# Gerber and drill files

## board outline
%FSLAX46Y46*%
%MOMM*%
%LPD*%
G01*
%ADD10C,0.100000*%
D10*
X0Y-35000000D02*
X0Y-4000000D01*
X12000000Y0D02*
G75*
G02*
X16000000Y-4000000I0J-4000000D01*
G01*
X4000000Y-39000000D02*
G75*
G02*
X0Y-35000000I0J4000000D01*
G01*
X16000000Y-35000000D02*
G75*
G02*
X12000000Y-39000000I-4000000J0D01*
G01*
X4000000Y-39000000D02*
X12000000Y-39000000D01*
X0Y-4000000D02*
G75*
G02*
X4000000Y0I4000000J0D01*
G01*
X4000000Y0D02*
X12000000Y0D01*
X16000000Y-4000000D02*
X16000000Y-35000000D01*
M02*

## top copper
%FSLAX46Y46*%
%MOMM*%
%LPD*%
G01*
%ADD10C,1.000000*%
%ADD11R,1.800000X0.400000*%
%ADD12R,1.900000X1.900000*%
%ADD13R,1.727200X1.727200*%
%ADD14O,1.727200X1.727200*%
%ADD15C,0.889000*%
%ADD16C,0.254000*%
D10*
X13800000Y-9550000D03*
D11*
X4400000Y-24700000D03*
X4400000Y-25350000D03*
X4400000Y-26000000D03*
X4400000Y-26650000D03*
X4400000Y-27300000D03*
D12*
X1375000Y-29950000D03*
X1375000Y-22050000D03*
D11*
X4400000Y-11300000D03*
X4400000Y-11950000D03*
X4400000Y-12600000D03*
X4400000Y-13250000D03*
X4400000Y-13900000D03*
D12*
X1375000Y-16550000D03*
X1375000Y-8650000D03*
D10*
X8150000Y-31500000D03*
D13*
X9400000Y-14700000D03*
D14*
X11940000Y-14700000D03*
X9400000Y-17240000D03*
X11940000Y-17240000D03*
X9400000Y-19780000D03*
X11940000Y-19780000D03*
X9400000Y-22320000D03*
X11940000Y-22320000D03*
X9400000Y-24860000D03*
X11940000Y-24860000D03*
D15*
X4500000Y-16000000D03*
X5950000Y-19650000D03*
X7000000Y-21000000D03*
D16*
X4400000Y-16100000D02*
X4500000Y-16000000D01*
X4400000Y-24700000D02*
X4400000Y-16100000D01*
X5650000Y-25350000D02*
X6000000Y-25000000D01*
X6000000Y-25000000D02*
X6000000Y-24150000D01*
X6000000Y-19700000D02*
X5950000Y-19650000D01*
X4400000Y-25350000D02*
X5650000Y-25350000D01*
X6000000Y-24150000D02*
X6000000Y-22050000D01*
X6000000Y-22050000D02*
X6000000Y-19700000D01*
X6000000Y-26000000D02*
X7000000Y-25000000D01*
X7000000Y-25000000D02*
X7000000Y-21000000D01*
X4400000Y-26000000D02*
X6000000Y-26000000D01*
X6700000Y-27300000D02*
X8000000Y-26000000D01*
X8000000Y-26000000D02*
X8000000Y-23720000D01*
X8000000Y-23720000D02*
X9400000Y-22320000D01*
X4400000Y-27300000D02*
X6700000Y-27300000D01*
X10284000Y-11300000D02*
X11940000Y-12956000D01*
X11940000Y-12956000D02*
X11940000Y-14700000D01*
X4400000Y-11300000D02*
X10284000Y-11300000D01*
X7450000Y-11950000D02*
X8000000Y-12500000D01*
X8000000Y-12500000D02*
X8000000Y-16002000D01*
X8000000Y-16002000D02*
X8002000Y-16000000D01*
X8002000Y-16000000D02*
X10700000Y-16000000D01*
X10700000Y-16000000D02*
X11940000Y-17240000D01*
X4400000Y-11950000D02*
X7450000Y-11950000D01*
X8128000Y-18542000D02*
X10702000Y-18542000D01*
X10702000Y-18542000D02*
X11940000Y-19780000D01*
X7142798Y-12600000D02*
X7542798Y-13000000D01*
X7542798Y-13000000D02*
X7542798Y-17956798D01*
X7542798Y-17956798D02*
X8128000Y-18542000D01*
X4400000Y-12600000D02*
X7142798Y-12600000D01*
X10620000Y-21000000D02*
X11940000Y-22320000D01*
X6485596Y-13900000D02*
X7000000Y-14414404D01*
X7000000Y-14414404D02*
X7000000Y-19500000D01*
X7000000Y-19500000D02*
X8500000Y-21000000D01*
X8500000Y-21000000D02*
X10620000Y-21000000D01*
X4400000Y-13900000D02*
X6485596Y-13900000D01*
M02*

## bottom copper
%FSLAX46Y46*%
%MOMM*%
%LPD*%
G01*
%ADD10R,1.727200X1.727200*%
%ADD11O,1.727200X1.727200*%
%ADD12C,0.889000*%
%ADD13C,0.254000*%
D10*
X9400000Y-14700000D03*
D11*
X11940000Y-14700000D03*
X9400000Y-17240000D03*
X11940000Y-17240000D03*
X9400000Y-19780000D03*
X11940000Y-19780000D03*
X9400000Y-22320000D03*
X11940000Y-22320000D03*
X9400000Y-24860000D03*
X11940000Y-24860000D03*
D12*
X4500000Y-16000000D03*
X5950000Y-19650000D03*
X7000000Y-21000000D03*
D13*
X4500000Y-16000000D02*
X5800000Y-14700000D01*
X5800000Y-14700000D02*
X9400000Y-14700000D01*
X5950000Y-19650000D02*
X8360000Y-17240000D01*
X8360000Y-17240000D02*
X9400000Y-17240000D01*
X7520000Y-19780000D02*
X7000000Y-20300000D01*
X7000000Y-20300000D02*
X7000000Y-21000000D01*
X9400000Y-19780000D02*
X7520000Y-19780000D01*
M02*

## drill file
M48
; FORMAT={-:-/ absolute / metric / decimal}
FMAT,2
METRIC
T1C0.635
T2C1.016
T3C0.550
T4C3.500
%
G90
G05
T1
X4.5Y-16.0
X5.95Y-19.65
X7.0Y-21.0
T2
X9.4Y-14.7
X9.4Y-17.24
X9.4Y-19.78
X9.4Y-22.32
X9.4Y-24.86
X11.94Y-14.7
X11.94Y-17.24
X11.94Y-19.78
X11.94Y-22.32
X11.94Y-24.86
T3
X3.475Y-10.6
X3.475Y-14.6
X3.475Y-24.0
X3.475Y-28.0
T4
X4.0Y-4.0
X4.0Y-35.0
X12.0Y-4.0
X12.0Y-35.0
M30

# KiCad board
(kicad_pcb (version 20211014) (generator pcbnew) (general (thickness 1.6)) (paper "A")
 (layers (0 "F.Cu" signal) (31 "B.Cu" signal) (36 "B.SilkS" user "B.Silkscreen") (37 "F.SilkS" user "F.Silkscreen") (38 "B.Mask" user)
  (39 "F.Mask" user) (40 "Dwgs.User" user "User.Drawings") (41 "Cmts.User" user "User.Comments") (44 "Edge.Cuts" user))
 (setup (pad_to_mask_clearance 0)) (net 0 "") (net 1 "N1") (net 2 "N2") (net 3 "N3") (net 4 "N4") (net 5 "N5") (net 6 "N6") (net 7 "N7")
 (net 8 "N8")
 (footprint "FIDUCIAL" (layer "F.Cu") (at 13.8 9.55)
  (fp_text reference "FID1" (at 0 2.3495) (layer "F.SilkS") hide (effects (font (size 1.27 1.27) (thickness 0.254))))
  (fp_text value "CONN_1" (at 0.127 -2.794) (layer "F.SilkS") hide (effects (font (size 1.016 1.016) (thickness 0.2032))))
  (pad "1" smd circle locked (at 0 0) (size 1 1) (layers "F.Cu" "F.Mask") (solder_mask_margin 1) (clearance 1)))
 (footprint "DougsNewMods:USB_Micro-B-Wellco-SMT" (layer "F.Cu") (at 4 26 -90)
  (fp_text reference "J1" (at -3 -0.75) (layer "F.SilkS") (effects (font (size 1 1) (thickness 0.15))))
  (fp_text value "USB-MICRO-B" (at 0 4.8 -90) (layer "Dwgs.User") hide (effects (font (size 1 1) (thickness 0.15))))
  (pad "" np_thru_hole circle locked (at 2 0.525) (size 0.55 0.55) (drill oval 0.55) (layers *.Cu *.Mask "F.SilkS"))
  (pad "" np_thru_hole circle locked (at -2 0.525) (size 0.55 0.55) (drill 0.55) (layers *.Cu *.Mask "F.SilkS"))
  (pad "1" smd rect locked (at -1.3 -0.4 270) (size 0.4 1.8) (layers "F.Cu" "F.Mask") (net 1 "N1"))
  (pad "2" smd rect locked (at -0.65 -0.4 270) (size 0.4 1.8) (layers "F.Cu" "F.Mask") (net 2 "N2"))
  (pad "3" smd rect locked (at 0 -0.4 270) (size 0.4 1.8) (layers "F.Cu" "F.Mask") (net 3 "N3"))
  (pad "4" smd rect locked (at 0.65 -0.4 270) (size 0.4 1.8) (layers "F.Cu" "F.Mask"))
  (pad "5" smd rect locked (at 1.3 -0.4 270) (size 0.4 1.8) (layers "F.Cu" "F.Mask") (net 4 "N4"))
  (pad "6" smd rect locked (at 3.95 2.625) (size 1.9 1.9) (layers "F.Cu" "F.Mask"))
  (pad "7" smd rect locked (at -3.95 2.625) (size 1.9 1.9) (layers "F.Cu" "F.Mask")))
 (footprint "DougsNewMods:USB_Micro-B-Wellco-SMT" (layer "F.Cu") (at 4 12.6 -90) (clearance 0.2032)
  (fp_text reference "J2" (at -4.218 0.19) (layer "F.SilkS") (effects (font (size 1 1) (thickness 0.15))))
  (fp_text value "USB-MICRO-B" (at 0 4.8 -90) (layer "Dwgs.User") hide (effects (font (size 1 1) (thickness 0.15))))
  (pad "" np_thru_hole circle locked (at -2 0.525) (size 0.55 0.55) (drill 0.55) (layers *.Cu *.Mask "F.SilkS"))
  (pad "" np_thru_hole circle locked (at 2 0.525) (size 0.55 0.55) (drill oval 0.55) (layers *.Cu *.Mask "F.SilkS"))
  (pad "1" smd rect locked (at -1.3 -0.4 270) (size 0.4 1.8) (layers "F.Cu" "F.Mask") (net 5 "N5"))
  (pad "2" smd rect locked (at -0.65 -0.4 270) (size 0.4 1.8) (layers "F.Cu" "F.Mask") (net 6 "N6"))
  (pad "3" smd rect locked (at 0 -0.4 270) (size 0.4 1.8) (layers "F.Cu" "F.Mask") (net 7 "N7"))
  (pad "4" smd rect locked (at 0.65 -0.4 270) (size 0.4 1.8) (layers "F.Cu" "F.Mask"))
  (pad "5" smd rect locked (at 1.3 -0.4 270) (size 0.4 1.8) (layers "F.Cu" "F.Mask") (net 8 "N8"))
  (pad "6" smd rect locked (at 3.95 2.625) (size 1.9 1.9) (layers "F.Cu" "F.Mask"))
  (pad "7" smd rect locked (at -3.95 2.625) (size 1.9 1.9) (layers "F.Cu" "F.Mask")))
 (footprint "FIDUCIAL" (layer "F.Cu") (at 8.15 31.5)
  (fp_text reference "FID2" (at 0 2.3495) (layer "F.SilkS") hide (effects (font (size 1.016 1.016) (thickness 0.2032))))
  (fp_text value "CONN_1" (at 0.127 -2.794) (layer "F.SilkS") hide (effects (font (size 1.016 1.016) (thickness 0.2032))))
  (pad "1" smd circle locked (at 0 0) (size 1 1) (layers "F.Cu" "F.Mask") (solder_mask_margin 1) (clearance 1)))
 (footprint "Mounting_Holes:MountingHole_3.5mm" (layer "F.Cu") (at 4 4)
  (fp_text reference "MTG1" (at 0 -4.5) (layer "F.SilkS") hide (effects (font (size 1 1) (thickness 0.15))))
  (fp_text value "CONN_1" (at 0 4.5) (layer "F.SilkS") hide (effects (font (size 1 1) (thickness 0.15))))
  (pad "" np_thru_hole circle locked (at 0 0) (size 3.5 3.5) (drill 3.5) (layers *.Cu *.Mask "F.SilkS")))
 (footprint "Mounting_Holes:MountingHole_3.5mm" (layer "F.Cu") (at 12 4)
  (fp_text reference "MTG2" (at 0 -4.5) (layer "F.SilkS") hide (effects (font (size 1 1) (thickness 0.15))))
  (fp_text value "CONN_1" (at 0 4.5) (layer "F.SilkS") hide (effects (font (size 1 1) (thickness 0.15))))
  (pad "" np_thru_hole circle locked (at 0 0) (size 3.5 3.5) (drill 3.5) (layers *.Cu *.Mask "F.SilkS")))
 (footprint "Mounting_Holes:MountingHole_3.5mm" (layer "F.Cu") (at 4 35)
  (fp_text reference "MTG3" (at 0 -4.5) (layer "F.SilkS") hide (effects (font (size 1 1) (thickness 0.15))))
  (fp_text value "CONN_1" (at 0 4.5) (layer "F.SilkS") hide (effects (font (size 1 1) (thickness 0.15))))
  (pad "" np_thru_hole circle locked (at 0 0) (size 3.5 3.5) (drill 3.5) (layers *.Cu *.Mask "F.SilkS")))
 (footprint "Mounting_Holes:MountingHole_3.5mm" (layer "F.Cu") (at 12 35)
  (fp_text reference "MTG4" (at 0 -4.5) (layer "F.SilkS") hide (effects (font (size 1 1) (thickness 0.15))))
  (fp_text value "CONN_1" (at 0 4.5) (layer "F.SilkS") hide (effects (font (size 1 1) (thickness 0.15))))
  (pad "" np_thru_hole circle locked (at 0 0) (size 3.5 3.5) (drill 3.5) (layers *.Cu *.Mask "F.SilkS")))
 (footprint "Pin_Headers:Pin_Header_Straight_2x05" (layer "F.Cu") (at 9.4 14.7)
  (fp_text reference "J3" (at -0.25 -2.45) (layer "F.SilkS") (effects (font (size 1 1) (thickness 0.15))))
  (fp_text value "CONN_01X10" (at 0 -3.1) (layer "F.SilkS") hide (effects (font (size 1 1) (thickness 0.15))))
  (pad "1" thru_hole rect locked (at 0 0) (size 1.7272 1.7272) (drill 1.016) (layers *.Cu *.Mask "F.SilkS") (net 1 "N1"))
  (pad "2" thru_hole oval locked (at 2.54 0) (size 1.7272 1.7272) (drill 1.016) (layers *.Cu *.Mask "F.SilkS") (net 5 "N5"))
  (pad "3" thru_hole oval locked (at 0 2.54) (size 1.7272 1.7272) (drill 1.016) (layers *.Cu *.Mask "F.SilkS") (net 2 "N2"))
  (pad "4" thru_hole oval locked (at 2.54 2.54) (size 1.7272 1.7272) (drill 1.016) (layers *.Cu *.Mask "F.SilkS") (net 6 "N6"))
  (pad "5" thru_hole oval locked (at 0 5.08) (size 1.7272 1.7272) (drill 1.016) (layers *.Cu *.Mask "F.SilkS") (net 3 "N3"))
  (pad "6" thru_hole oval locked (at 2.54 5.08) (size 1.7272 1.7272) (drill 1.016) (layers *.Cu *.Mask "F.SilkS") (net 7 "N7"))
  (pad "7" thru_hole oval locked (at 0 7.62) (size 1.7272 1.7272) (drill 1.016) (layers *.Cu *.Mask "F.SilkS") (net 4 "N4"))
  (pad "8" thru_hole oval locked (at 2.54 7.62) (size 1.7272 1.7272) (drill 1.016) (layers *.Cu *.Mask "F.SilkS") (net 8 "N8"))
  (pad "9" thru_hole oval locked (at 0 10.16) (size 1.7272 1.7272) (drill 1.016) (layers *.Cu *.Mask "F.SilkS"))
  (pad "10" thru_hole oval locked (at 2.54 10.16) (size 1.7272 1.7272) (drill 1.016) (layers *.Cu *.Mask "F.SilkS")))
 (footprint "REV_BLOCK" (layer "B.Cu") (at 13.15 10.8)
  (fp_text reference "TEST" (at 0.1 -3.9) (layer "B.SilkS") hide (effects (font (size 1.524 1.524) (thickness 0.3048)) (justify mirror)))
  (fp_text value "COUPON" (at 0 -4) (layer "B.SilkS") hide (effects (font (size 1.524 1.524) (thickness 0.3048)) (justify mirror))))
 (gr_line (start 0 35) (end 0 4) (layer "Edge.Cuts") (width 0.1))
 (gr_arc (start 12 0) (mid 14.828427 1.171573) (end 16 4) (layer "Edge.Cuts") (width 0.1))
 (gr_arc (start 4 39) (mid 1.171573 37.828427) (end 0 35) (layer "Edge.Cuts") (width 0.1))
 (gr_arc (start 16 35) (mid 14.828427 37.828427) (end 12 39) (layer "Edge.Cuts") (width 0.1))
 (gr_line (start 4 39) (end 12 39) (layer "Edge.Cuts") (width 0.1))
 (gr_arc (start 0 4) (mid 1.171573 1.171573) (end 4 0) (layer "Edge.Cuts") (width 0.1))
 (gr_line (start 4 0) (end 12 0) (layer "Edge.Cuts") (width 0.1))
 (gr_line (start 16 4) (end 16 35) (layer "Edge.Cuts") (width 0.1))
 (segment (start 4.4 16.1) (end 4.5 16) (width 0.254) (layer "F.Cu") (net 1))
 (segment (start 4.4 24.7) (end 4.4 16.1) (width 0.254) (layer "F.Cu") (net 1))
 (via (at 4.5 16) (size 0.889) (drill 0.635) (layers "F.Cu" "B.Cu") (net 1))
 (segment (start 4.5 16) (end 5.8 14.7) (width 0.254) (layer "B.Cu") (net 1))
 (segment (start 5.8 14.7) (end 9.4 14.7) (width 0.254) (layer "B.Cu") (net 1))
 (segment (start 5.65 25.35) (end 6 25) (width 0.254) (layer "F.Cu") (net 2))
 (segment (start 6 25) (end 6 24.15) (width 0.254) (layer "F.Cu") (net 2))
 (segment (start 6 19.7) (end 5.95 19.65) (width 0.254) (layer "F.Cu") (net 2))
 (segment (start 4.4 25.35) (end 5.65 25.35) (width 0.254) (layer "F.Cu") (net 2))
 (segment (start 6 24.15) (end 6 22.05) (width 0.254) (layer "F.Cu") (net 2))
 (segment (start 6 22.05) (end 6 19.7) (width 0.254) (layer "F.Cu") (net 2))
 (via (at 5.95 19.65) (size 0.889) (drill 0.635) (layers "F.Cu" "B.Cu") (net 2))
 (segment (start 5.95 19.65) (end 8.36 17.24) (width 0.254) (layer "B.Cu") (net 2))
 (segment (start 8.36 17.24) (end 9.4 17.24) (width 0.254) (layer "B.Cu") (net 2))
 (segment (start 6 26) (end 7 25) (width 0.254) (layer "F.Cu") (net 3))
 (segment (start 7 25) (end 7 21) (width 0.254) (layer "F.Cu") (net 3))
 (segment (start 4.4 26) (end 6 26) (width 0.254) (layer "F.Cu") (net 3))
 (via (at 7 21) (size 0.889) (drill 0.635) (layers "F.Cu" "B.Cu") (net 3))
 (segment (start 7.52 19.78) (end 7 20.3) (width 0.254) (layer "B.Cu") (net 3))
 (segment (start 7 20.3) (end 7 21) (width 0.254) (layer "B.Cu") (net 3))
 (segment (start 9.4 19.78) (end 7.52 19.78) (width 0.254) (layer "B.Cu") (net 3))
 (segment (start 6.7 27.3) (end 8 26) (width 0.254) (layer "F.Cu") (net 4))
 (segment (start 8 26) (end 8 23.72) (width 0.254) (layer "F.Cu") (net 4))
 (segment (start 8 23.72) (end 9.4 22.32) (width 0.254) (layer "F.Cu") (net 4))
 (segment (start 4.4 27.3) (end 6.7 27.3) (width 0.254) (layer "F.Cu") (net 4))
 (segment (start 10.284 11.3) (end 11.94 12.956) (width 0.254) (layer "F.Cu") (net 5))
 (segment (start 11.94 12.956) (end 11.94 14.7) (width 0.254) (layer "F.Cu") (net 5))
 (segment (start 4.4 11.3) (end 10.284 11.3) (width 0.254) (layer "F.Cu") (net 5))
 (segment (start 7.45 11.95) (end 8 12.5) (width 0.254) (layer "F.Cu") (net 6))
 (segment (start 8 12.5) (end 8 16.002) (width 0.254) (layer "F.Cu") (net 6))
 (segment (start 8 16.002) (end 8.002 16) (width 0.254) (layer "F.Cu") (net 6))
 (segment (start 8.002 16) (end 10.7 16) (width 0.254) (layer "F.Cu") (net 6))
 (segment (start 10.7 16) (end 11.94 17.24) (width 0.254) (layer "F.Cu") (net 6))
 (segment (start 4.4 11.95) (end 7.45 11.95) (width 0.254) (layer "F.Cu") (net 6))
 (segment (start 8.128 18.542) (end 10.702 18.542) (width 0.254) (layer "F.Cu") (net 7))
 (segment (start 10.702 18.542) (end 11.94 19.78) (width 0.254) (layer "F.Cu") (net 7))
 (segment (start 7.142798 12.6) (end 7.542798 13) (width 0.254) (layer "F.Cu") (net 7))
 (segment (start 7.542798 13) (end 7.542798 17.956798) (width 0.254) (layer "F.Cu") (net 7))
 (segment (start 7.542798 17.956798) (end 8.128 18.542) (width 0.254) (layer "F.Cu") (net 7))
 (segment (start 4.4 12.6) (end 7.142798 12.6) (width 0.254) (layer "F.Cu") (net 7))
 (segment (start 10.62 21) (end 11.94 22.32) (width 0.254) (layer "F.Cu") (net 8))
 (segment (start 6.485596 13.9) (end 7 14.414404) (width 0.254) (layer "F.Cu") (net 8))
 (segment (start 7 14.414404) (end 7 19.5) (width 0.254) (layer "F.Cu") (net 8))
 (segment (start 7 19.5) (end 8.5 21) (width 0.254) (layer "F.Cu") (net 8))
 (segment (start 8.5 21) (end 10.62 21) (width 0.254) (layer "F.Cu") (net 8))
 (segment (start 4.4 13.9) (end 6.485596 13.9) (width 0.254) (layer "F.Cu") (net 8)))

